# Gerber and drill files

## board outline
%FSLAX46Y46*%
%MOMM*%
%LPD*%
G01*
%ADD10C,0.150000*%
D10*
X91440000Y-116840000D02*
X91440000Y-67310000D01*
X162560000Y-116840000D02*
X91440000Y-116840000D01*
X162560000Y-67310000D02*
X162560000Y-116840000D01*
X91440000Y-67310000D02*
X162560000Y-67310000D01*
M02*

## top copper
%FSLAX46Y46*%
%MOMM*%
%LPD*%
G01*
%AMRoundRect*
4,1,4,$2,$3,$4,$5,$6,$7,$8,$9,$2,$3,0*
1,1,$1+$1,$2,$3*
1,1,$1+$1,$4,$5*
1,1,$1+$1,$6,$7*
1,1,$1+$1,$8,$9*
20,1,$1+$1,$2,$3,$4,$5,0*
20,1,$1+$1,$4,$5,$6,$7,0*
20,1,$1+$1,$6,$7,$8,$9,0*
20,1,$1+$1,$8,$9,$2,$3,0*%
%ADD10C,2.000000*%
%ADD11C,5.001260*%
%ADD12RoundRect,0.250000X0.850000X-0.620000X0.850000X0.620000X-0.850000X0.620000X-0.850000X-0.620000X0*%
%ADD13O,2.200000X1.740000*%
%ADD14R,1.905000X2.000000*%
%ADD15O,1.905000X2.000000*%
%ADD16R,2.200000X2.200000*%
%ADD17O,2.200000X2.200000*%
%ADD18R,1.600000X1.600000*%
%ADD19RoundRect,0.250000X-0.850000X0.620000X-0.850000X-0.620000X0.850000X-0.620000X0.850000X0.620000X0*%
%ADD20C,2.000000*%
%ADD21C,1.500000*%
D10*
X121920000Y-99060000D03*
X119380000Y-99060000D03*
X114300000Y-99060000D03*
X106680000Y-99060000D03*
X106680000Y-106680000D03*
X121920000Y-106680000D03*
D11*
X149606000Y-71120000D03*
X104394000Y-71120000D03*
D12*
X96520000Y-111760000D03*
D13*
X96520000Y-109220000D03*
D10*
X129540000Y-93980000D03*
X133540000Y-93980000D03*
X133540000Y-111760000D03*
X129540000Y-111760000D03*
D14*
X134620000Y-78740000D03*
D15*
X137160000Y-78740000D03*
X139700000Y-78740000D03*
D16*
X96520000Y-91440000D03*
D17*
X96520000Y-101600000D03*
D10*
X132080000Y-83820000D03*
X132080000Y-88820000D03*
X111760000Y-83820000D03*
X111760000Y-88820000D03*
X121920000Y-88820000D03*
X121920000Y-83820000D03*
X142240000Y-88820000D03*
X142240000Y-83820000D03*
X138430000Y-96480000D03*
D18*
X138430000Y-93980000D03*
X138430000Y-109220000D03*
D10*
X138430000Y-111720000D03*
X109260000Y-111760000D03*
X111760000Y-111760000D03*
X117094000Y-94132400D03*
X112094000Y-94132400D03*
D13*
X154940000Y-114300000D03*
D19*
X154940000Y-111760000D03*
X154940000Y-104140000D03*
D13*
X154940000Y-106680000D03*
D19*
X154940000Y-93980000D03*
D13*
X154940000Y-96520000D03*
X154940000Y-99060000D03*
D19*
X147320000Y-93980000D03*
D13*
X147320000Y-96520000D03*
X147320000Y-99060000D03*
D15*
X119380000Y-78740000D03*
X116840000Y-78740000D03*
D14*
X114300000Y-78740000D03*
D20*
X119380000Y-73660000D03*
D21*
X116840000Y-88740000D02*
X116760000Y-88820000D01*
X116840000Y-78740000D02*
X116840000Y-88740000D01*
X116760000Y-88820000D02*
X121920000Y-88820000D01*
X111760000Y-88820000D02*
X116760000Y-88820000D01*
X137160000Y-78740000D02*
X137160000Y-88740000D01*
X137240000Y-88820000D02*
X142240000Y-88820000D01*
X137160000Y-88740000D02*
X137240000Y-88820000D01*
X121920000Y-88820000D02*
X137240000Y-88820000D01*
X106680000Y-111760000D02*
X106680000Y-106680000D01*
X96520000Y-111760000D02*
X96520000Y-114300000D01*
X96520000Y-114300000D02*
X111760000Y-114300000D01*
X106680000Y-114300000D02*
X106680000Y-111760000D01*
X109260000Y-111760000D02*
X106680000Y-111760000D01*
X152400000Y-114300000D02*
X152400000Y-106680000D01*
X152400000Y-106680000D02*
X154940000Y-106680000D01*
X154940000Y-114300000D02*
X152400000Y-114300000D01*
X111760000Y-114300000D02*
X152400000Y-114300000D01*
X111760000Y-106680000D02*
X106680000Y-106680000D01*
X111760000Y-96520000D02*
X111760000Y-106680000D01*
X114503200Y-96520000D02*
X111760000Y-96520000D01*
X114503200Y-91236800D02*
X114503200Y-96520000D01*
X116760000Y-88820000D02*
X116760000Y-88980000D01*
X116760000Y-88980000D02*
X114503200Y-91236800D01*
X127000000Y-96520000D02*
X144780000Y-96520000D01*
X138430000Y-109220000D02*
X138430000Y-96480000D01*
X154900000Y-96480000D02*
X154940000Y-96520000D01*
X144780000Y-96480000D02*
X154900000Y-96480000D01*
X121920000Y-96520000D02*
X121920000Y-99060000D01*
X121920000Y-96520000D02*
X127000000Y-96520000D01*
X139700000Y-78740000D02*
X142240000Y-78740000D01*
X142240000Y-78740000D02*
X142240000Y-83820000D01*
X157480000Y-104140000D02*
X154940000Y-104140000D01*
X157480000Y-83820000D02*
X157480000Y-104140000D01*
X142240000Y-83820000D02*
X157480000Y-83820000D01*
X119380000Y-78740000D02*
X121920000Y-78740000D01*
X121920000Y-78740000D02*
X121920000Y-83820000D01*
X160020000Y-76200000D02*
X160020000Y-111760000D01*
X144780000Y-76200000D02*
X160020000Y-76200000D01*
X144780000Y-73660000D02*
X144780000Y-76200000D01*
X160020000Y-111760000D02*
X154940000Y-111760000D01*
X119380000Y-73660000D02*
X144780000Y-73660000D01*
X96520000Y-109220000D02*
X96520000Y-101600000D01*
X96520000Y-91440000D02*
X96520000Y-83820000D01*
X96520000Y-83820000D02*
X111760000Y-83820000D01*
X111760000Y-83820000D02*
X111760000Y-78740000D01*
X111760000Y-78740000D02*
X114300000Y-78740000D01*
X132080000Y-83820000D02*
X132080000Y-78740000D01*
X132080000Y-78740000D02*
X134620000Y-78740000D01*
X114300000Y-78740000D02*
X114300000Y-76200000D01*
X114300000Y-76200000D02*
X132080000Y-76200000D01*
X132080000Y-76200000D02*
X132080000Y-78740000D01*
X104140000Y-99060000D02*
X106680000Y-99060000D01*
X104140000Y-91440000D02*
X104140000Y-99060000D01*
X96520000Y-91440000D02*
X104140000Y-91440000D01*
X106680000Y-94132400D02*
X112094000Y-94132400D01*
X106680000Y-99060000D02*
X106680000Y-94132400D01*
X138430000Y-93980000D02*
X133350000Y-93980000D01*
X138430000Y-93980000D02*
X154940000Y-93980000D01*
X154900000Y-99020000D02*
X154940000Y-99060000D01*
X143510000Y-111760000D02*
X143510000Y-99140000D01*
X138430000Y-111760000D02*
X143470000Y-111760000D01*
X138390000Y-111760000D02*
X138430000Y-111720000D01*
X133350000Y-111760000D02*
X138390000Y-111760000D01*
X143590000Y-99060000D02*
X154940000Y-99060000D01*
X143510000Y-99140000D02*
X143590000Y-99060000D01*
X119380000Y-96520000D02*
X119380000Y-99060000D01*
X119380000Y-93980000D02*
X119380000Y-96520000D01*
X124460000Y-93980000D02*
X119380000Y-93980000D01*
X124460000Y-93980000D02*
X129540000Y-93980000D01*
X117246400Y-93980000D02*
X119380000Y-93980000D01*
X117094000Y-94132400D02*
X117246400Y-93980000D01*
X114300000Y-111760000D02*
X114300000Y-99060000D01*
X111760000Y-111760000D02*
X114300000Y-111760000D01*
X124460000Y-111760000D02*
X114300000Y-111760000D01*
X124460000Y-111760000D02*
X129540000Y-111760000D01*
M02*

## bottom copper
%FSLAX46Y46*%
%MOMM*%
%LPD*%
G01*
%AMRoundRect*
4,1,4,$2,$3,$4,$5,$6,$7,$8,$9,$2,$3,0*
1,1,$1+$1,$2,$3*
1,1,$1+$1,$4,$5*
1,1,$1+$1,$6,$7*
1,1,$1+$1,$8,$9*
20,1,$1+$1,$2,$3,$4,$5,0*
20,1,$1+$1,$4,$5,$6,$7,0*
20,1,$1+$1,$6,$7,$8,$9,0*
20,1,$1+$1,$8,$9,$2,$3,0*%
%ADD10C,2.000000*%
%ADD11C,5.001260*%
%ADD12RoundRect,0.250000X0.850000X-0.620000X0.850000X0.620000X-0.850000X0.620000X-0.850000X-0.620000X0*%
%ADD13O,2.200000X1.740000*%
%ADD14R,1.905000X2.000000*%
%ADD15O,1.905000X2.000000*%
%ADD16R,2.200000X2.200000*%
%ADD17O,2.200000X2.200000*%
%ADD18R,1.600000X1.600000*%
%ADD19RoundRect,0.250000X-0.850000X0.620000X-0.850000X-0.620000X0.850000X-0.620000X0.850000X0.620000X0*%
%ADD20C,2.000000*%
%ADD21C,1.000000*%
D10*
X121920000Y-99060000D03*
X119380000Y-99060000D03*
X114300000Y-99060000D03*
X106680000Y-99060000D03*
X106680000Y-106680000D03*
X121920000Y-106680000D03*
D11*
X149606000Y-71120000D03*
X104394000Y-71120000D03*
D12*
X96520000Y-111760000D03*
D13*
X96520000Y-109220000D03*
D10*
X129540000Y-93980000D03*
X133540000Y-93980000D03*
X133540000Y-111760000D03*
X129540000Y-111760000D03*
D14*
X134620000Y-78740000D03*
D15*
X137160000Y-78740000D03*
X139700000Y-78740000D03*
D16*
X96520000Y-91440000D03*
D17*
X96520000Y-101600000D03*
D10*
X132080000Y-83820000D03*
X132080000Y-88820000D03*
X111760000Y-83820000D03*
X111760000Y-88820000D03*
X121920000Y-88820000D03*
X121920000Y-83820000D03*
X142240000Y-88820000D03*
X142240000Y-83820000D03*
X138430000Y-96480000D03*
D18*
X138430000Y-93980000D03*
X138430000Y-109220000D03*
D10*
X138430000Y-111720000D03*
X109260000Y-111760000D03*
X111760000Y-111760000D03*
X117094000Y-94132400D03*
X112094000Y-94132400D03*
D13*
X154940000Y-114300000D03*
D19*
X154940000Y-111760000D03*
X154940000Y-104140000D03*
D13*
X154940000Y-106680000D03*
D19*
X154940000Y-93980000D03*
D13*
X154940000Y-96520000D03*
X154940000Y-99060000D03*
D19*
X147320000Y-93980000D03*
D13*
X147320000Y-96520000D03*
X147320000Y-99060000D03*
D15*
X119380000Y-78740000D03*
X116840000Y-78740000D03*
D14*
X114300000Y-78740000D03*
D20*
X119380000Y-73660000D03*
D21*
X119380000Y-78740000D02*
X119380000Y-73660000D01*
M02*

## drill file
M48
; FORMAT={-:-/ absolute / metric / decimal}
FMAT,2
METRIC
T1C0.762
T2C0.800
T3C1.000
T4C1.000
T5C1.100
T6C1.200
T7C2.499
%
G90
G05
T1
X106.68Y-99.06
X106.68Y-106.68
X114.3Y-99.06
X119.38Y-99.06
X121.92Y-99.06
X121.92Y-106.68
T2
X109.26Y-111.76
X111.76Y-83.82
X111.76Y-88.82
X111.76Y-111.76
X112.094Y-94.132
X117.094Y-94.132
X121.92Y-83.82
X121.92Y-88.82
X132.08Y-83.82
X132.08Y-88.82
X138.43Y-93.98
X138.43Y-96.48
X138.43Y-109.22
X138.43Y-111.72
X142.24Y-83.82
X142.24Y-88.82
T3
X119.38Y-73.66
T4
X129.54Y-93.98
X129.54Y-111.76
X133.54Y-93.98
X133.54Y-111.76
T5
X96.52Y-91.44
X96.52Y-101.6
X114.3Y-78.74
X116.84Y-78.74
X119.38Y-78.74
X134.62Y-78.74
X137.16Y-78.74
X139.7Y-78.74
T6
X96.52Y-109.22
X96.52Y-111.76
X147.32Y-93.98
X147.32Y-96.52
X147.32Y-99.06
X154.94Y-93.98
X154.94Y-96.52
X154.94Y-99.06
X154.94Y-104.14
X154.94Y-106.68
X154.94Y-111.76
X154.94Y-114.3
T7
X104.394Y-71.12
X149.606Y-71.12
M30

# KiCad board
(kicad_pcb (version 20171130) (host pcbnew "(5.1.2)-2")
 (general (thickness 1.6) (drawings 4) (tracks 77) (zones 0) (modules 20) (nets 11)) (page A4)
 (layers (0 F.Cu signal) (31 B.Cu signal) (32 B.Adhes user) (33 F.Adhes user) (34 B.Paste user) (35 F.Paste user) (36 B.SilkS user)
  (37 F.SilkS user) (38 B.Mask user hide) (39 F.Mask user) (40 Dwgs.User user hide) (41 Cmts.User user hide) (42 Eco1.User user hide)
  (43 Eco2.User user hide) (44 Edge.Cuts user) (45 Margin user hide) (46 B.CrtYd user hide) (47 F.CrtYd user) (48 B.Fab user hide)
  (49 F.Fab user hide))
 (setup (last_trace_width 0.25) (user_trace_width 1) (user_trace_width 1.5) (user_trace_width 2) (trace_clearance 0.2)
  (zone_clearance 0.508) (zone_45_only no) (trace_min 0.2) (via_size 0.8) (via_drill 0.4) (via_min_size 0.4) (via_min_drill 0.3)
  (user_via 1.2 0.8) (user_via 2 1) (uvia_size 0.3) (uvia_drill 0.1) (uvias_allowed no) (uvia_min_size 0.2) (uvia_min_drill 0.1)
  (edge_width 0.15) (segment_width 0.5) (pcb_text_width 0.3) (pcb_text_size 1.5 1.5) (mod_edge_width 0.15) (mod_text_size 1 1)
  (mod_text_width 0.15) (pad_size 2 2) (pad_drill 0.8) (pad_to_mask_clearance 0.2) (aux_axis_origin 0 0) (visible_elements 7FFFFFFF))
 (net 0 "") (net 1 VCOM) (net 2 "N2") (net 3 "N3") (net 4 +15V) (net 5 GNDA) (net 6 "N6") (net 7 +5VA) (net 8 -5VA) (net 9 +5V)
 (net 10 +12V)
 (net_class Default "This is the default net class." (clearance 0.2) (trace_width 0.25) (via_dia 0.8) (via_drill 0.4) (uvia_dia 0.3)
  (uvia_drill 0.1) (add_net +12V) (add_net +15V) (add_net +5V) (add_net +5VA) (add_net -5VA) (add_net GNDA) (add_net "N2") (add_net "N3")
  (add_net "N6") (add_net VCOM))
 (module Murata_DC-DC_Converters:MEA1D (layer F.Cu) (at 114.3 104.14)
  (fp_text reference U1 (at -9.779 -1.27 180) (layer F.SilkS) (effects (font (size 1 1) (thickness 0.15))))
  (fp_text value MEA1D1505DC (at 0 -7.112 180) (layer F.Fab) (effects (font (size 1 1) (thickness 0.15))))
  (pad 8 thru_hole circle (at 7.62 -5.08) (size 2 2) (drill 0.762) (layers *.Cu *.Mask) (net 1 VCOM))
  (pad 9 thru_hole circle (at 5.08 -5.08) (size 2 2) (drill 0.762) (layers *.Cu *.Mask) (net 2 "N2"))
  (pad 11 thru_hole circle (at 0 -5.08) (size 2 2) (drill 0.762) (layers *.Cu *.Mask) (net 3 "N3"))
  (pad 14 thru_hole circle (at -7.62 -5.08) (size 2 2) (drill 0.762) (layers *.Cu *.Mask) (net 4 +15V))
  (pad 1 thru_hole circle (at -7.62 2.54) (size 2 2) (drill 0.762) (layers *.Cu *.Mask) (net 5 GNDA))
  (pad 7 thru_hole circle (at 7.62 2.54) (size 2 2) (drill 0.762) (layers *.Cu *.Mask)))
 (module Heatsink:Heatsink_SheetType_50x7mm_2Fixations (layer F.Cu) (at 127 71.12) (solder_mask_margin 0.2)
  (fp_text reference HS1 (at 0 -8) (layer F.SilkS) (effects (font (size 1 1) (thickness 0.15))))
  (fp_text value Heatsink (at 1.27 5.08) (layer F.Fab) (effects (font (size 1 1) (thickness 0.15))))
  (pad 1 thru_hole circle (at 22.606 0) (size 5.00126 5.00126) (drill 2.49936) (layers *.Cu *.Mask))
  (pad 1 thru_hole circle (at -22.606 0) (size 5.00126 5.00126) (drill 2.49936) (layers *.Cu *.Mask)))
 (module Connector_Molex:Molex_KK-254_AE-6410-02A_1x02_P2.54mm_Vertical (layer F.Cu) (at 96.52 111.76 90)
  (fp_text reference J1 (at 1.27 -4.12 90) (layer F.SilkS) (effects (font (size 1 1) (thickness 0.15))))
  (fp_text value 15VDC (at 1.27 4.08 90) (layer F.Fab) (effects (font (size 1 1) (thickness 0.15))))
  (pad 1 thru_hole roundrect (at 0 0 90) (size 1.74 2.2) (drill 1.2) (layers *.Cu *.Mask) (roundrect_rratio 0.143678) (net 5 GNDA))
  (pad 2 thru_hole oval (at 2.54 0 90) (size 1.74 2.2) (drill 1.2) (layers *.Cu *.Mask) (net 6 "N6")))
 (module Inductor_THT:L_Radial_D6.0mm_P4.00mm (layer F.Cu) (at 129.54 93.98)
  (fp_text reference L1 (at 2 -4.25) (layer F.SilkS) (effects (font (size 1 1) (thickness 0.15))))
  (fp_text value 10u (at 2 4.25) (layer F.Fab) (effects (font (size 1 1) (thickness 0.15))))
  (pad 1 thru_hole circle (at 0 0) (size 2 2) (drill 1) (layers *.Cu *.Mask) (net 2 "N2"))
  (pad 2 thru_hole circle (at 4 0) (size 2 2) (drill 1) (layers *.Cu *.Mask) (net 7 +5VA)))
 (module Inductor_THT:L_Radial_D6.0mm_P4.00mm (layer F.Cu) (at 129.54 111.76)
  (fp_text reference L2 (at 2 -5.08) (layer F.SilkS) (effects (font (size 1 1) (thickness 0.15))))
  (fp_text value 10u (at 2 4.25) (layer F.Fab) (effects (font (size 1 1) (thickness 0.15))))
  (pad 2 thru_hole circle (at 4 0) (size 2 2) (drill 1) (layers *.Cu *.Mask) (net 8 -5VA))
  (pad 1 thru_hole circle (at 0 0) (size 2 2) (drill 1) (layers *.Cu *.Mask) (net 3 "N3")))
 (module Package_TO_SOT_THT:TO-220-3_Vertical (layer F.Cu) (at 134.62 78.74)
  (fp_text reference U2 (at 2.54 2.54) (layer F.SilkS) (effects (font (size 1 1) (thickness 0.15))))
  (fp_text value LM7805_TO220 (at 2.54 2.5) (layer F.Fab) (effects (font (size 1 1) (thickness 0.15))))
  (pad 1 thru_hole rect (at 0 0) (size 1.905 2) (drill 1.1) (layers *.Cu *.Mask) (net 4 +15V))
  (pad 2 thru_hole oval (at 2.54 0) (size 1.905 2) (drill 1.1) (layers *.Cu *.Mask) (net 5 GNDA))
  (pad 3 thru_hole oval (at 5.08 0) (size 1.905 2) (drill 1.1) (layers *.Cu *.Mask) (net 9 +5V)))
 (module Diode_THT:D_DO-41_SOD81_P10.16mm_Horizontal (layer F.Cu) (at 96.52 91.44 270)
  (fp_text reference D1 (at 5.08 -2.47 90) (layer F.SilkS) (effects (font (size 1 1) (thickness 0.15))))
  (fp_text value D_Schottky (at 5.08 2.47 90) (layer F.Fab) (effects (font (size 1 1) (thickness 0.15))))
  (pad 1 thru_hole rect (at 0 0 270) (size 2.2 2.2) (drill 1.1) (layers *.Cu *.Mask) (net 4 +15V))
  (pad 2 thru_hole oval (at 10.16 0 270) (size 2.2 2.2) (drill 1.1) (layers *.Cu *.Mask) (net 6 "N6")))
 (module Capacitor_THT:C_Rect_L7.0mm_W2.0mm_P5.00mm (layer F.Cu) (at 132.08 83.82 270)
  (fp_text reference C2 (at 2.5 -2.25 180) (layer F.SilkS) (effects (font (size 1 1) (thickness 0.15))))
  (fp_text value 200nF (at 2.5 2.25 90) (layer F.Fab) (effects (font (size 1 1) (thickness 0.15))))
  (pad 1 thru_hole circle (at 0 0 270) (size 2 2) (drill 0.8) (layers *.Cu *.Mask) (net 4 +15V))
  (pad 2 thru_hole circle (at 5 0 270) (size 2 2) (drill 0.8) (layers *.Cu *.Mask) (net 5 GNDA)))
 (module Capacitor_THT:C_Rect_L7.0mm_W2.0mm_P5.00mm (layer F.Cu) (at 111.76 83.82 270)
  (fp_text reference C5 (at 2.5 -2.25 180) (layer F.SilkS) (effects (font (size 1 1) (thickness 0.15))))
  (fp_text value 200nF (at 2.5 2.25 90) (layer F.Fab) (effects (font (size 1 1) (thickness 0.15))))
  (pad 1 thru_hole circle (at 0 0 270) (size 2 2) (drill 0.8) (layers *.Cu *.Mask) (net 4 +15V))
  (pad 2 thru_hole circle (at 5 0 270) (size 2 2) (drill 0.8) (layers *.Cu *.Mask) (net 5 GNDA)))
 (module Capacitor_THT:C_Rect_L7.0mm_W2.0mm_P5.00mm (layer F.Cu) (at 121.92 83.82 270)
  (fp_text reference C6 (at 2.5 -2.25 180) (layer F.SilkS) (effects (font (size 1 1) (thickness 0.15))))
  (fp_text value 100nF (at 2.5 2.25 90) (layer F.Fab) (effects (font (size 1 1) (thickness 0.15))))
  (pad 2 thru_hole circle (at 5 0 270) (size 2 2) (drill 0.8) (layers *.Cu *.Mask) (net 5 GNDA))
  (pad 1 thru_hole circle (at 0 0 270) (size 2 2) (drill 0.8) (layers *.Cu *.Mask) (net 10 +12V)))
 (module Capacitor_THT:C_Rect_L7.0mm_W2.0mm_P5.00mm (layer F.Cu) (at 142.24 83.82 270)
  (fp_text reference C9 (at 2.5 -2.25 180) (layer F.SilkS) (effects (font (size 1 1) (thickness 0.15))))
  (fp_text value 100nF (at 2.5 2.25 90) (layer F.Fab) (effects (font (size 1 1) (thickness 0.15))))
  (pad 2 thru_hole circle (at 5 0 270) (size 2 2) (drill 0.8) (layers *.Cu *.Mask) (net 5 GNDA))
  (pad 1 thru_hole circle (at 0 0 270) (size 2 2) (drill 0.8) (layers *.Cu *.Mask) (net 9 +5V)))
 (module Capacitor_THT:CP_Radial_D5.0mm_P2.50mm (layer F.Cu) (at 138.43 93.98 270)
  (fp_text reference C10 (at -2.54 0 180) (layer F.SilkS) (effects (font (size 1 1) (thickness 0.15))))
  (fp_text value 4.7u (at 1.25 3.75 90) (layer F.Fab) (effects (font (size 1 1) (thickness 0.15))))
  (pad 2 thru_hole circle (at 2.5 0 270) (size 2 2) (drill 0.8) (layers *.Cu *.Mask) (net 1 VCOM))
  (pad 1 thru_hole rect (at 0 0 270) (size 1.6 1.6) (drill 0.8) (layers *.Cu *.Mask) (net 7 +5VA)))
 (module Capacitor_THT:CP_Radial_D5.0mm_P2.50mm (layer F.Cu) (at 138.43 109.22 270)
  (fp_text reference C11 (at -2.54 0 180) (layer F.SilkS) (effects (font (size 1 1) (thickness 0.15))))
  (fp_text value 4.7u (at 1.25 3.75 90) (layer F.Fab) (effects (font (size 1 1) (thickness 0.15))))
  (pad 1 thru_hole rect (at 0 0 270) (size 1.6 1.6) (drill 0.8) (layers *.Cu *.Mask) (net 1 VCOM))
  (pad 2 thru_hole circle (at 2.5 0 270) (size 2 2) (drill 0.8) (layers *.Cu *.Mask) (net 8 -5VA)))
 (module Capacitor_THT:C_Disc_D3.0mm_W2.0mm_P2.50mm (layer F.Cu) (at 111.76 111.76 180)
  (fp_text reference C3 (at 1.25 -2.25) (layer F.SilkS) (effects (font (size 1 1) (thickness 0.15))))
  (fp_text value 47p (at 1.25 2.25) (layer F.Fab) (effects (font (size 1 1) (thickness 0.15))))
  (pad 2 thru_hole circle (at 2.5 0 180) (size 2 2) (drill 0.8) (layers *.Cu *.Mask) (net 5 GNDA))
  (pad 1 thru_hole circle (at 0 0 180) (size 2 2) (drill 0.8) (layers *.Cu *.Mask) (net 3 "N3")))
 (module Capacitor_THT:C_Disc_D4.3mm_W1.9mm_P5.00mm (layer F.Cu) (at 117.094 94.1324 180)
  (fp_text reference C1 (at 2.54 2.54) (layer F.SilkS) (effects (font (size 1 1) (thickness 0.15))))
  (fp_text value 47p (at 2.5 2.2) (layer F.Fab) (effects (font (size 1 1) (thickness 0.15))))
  (pad 1 thru_hole circle (at 0 0 180) (size 2 2) (drill 0.8) (layers *.Cu *.Mask) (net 2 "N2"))
  (pad 2 thru_hole circle (at 5 0 180) (size 2 2) (drill 0.8) (layers *.Cu *.Mask) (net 4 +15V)))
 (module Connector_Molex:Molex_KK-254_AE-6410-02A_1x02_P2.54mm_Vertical (layer F.Cu) (at 154.94 111.76 270)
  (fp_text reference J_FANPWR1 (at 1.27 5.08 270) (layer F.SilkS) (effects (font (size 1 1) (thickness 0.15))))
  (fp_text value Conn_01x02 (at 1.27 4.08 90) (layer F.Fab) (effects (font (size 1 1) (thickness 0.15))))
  (pad 2 thru_hole oval (at 2.54 0 270) (size 1.74 2.2) (drill 1.2) (layers *.Cu *.Mask) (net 5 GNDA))
  (pad 1 thru_hole roundrect (at 0 0 270) (size 1.74 2.2) (drill 1.2) (layers *.Cu *.Mask) (roundrect_rratio 0.143678) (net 10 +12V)))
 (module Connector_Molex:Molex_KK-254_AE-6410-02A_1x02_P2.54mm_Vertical (layer F.Cu) (at 154.94 104.14 270)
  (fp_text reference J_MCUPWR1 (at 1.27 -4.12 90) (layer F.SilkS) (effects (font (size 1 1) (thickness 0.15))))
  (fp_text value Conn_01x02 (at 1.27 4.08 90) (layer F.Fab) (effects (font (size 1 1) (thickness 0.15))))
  (pad 1 thru_hole roundrect (at 0 0 270) (size 1.74 2.2) (drill 1.2) (layers *.Cu *.Mask) (roundrect_rratio 0.143678) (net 9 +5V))
  (pad 2 thru_hole oval (at 2.54 0 270) (size 1.74 2.2) (drill 1.2) (layers *.Cu *.Mask) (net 5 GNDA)))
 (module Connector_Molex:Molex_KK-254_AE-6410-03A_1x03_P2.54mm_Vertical (layer F.Cu) (at 154.94 93.98 270)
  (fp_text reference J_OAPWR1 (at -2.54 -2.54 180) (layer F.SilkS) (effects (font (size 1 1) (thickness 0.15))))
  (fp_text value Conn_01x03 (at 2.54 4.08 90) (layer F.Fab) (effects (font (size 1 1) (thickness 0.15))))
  (pad 1 thru_hole roundrect (at 0 0 270) (size 1.74 2.2) (drill 1.2) (layers *.Cu *.Mask) (roundrect_rratio 0.143678) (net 7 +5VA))
  (pad 2 thru_hole oval (at 2.54 0 270) (size 1.74 2.2) (drill 1.2) (layers *.Cu *.Mask) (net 1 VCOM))
  (pad 3 thru_hole oval (at 5.08 0 270) (size 1.74 2.2) (drill 1.2) (layers *.Cu *.Mask) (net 8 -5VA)))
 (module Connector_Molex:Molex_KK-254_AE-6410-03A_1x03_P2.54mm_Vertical (layer F.Cu) (at 147.32 93.98 270)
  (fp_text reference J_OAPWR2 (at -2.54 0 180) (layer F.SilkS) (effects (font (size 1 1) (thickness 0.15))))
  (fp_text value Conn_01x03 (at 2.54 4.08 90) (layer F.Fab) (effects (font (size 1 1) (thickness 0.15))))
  (pad 1 thru_hole roundrect (at 0 0 270) (size 1.74 2.2) (drill 1.2) (layers *.Cu *.Mask) (roundrect_rratio 0.143678) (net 7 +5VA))
  (pad 2 thru_hole oval (at 2.54 0 270) (size 1.74 2.2) (drill 1.2) (layers *.Cu *.Mask) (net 1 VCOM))
  (pad 3 thru_hole oval (at 5.08 0 270) (size 1.74 2.2) (drill 1.2) (layers *.Cu *.Mask) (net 8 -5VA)))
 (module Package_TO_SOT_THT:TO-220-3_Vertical (layer F.Cu) (at 114.3 78.74)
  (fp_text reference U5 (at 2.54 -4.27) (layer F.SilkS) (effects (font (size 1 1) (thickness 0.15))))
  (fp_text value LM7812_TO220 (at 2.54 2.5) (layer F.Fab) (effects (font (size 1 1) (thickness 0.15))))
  (pad 3 thru_hole oval (at 5.08 0) (size 1.905 2) (drill 1.1) (layers *.Cu *.Mask) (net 10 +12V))
  (pad 2 thru_hole oval (at 2.54 0) (size 1.905 2) (drill 1.1) (layers *.Cu *.Mask) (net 5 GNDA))
  (pad 1 thru_hole rect (at 0 0) (size 1.905 2) (drill 1.1) (layers *.Cu *.Mask) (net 4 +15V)))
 (gr_line (start 91.44 116.84) (end 91.44 67.31) (layer Edge.Cuts) (width 0.15))
 (gr_line (start 162.56 116.84) (end 91.44 116.84) (layer Edge.Cuts) (width 0.15))
 (gr_line (start 162.56 67.31) (end 162.56 116.84) (layer Edge.Cuts) (width 0.15))
 (gr_line (start 91.44 67.31) (end 162.56 67.31) (layer Edge.Cuts) (width 0.15))
 (segment (start 116.84 88.74) (end 116.76 88.82) (width 1.5) (layer F.Cu) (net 5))
 (segment (start 116.84 78.74) (end 116.84 88.74) (width 1.5) (layer F.Cu) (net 5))
 (segment (start 116.76 88.82) (end 121.92 88.82) (width 1.5) (layer F.Cu) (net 5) (status 20))
 (segment (start 111.76 88.82) (end 116.76 88.82) (width 1.5) (layer F.Cu) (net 5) (status 10))
 (segment (start 137.16 78.74) (end 137.16 88.74) (width 1.5) (layer F.Cu) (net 5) (status 10))
 (segment (start 137.24 88.82) (end 142.24 88.82) (width 1.5) (layer F.Cu) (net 5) (status 20))
 (segment (start 137.16 88.74) (end 137.24 88.82) (width 1.5) (layer F.Cu) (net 5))
 (segment (start 121.92 88.82) (end 137.24 88.82) (width 1.5) (layer F.Cu) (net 5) (status 10))
 (segment (start 106.68 111.76) (end 106.68 106.68) (width 1.5) (layer F.Cu) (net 5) (status 20))
 (segment (start 96.52 111.76) (end 96.52 114.3) (width 1.5) (layer F.Cu) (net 5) (status 10))
 (segment (start 96.52 114.3) (end 111.76 114.3) (width 1.5) (layer F.Cu) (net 5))
 (segment (start 106.68 114.3) (end 106.68 111.76) (width 1.5) (layer F.Cu) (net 5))
 (segment (start 109.26 111.76) (end 106.68 111.76) (width 1.5) (layer F.Cu) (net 5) (status 10))
 (segment (start 152.4 114.3) (end 152.4 106.68) (width 1.5) (layer F.Cu) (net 5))
 (segment (start 152.4 106.68) (end 154.94 106.68) (width 1.5) (layer F.Cu) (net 5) (status 20))
 (segment (start 154.94 114.3) (end 152.4 114.3) (width 1.5) (layer F.Cu) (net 5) (status 10))
 (segment (start 111.76 114.3) (end 152.4 114.3) (width 1.5) (layer F.Cu) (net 5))
 (segment (start 111.76 106.68) (end 106.68 106.68) (width 1.5) (layer F.Cu) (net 5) (status 20))
 (segment (start 111.76 96.52) (end 111.76 106.68) (width 1.5) (layer F.Cu) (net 5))
 (segment (start 114.5032 96.52) (end 111.76 96.52) (width 1.5) (layer F.Cu) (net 5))
 (segment (start 114.5032 91.2368) (end 114.5032 96.52) (width 1.5) (layer F.Cu) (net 5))
 (segment (start 116.76 88.82) (end 116.76 88.98) (width 1.5) (layer F.Cu) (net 5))
 (segment (start 116.76 88.98) (end 114.5032 91.2368) (width 1.5) (layer F.Cu) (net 5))
 (segment (start 127 96.52) (end 144.78 96.52) (width 1.5) (layer F.Cu) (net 1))
 (segment (start 138.43 109.22) (end 138.43 96.48) (width 1.5) (layer F.Cu) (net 1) (status 30))
 (segment (start 154.9 96.48) (end 154.94 96.52) (width 1.5) (layer F.Cu) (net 1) (status 30))
 (segment (start 144.78 96.48) (end 154.9 96.48) (width 1.5) (layer F.Cu) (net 1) (status 20))
 (segment (start 121.92 96.52) (end 121.92 99.06) (width 1.5) (layer F.Cu) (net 1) (status 20))
 (segment (start 121.92 96.52) (end 127 96.52) (width 1.5) (layer F.Cu) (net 1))
 (segment (start 139.7 78.74) (end 142.24 78.74) (width 1.5) (layer F.Cu) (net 9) (status 10))
 (segment (start 142.24 78.74) (end 142.24 83.82) (width 1.5) (layer F.Cu) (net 9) (status 20))
 (segment (start 157.48 104.14) (end 154.94 104.14) (width 1.5) (layer F.Cu) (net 9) (status 20))
 (segment (start 157.48 83.82) (end 157.48 104.14) (width 1.5) (layer F.Cu) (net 9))
 (segment (start 142.24 83.82) (end 157.48 83.82) (width 1.5) (layer F.Cu) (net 9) (status 10))
 (segment (start 119.38 78.74) (end 121.92 78.74) (width 1.5) (layer F.Cu) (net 10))
 (segment (start 121.92 78.74) (end 121.92 83.82) (width 1.5) (layer F.Cu) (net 10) (status 20))
 (segment (start 119.38 78.74) (end 119.38 73.66) (width 1) (layer B.Cu) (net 10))
 (via (at 119.38 73.66) (size 2) (drill 1) (layers F.Cu B.Cu) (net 10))
 (segment (start 160.02 76.2) (end 160.02 111.76) (width 1.5) (layer F.Cu) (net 10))
 (segment (start 144.78 76.2) (end 160.02 76.2) (width 1.5) (layer F.Cu) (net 10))
 (segment (start 144.78 73.66) (end 144.78 76.2) (width 1.5) (layer F.Cu) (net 10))
 (segment (start 160.02 111.76) (end 154.94 111.76) (width 1.5) (layer F.Cu) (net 10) (status 20))
 (segment (start 119.38 73.66) (end 144.78 73.66) (width 1.5) (layer F.Cu) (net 10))
 (segment (start 96.52 109.22) (end 96.52 101.6) (width 1.5) (layer F.Cu) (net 6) (status 30))
 (segment (start 96.52 91.44) (end 96.52 83.82) (width 1.5) (layer F.Cu) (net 4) (status 10))
 (segment (start 96.52 83.82) (end 111.76 83.82) (width 1.5) (layer F.Cu) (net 4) (status 20))
 (segment (start 111.76 83.82) (end 111.76 78.74) (width 1.5) (layer F.Cu) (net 4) (status 10))
 (segment (start 111.76 78.74) (end 114.3 78.74) (width 1.5) (layer F.Cu) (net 4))
 (segment (start 132.08 83.82) (end 132.08 78.74) (width 1.5) (layer F.Cu) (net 4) (status 10))
 (segment (start 132.08 78.74) (end 134.62 78.74) (width 1.5) (layer F.Cu) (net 4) (status 20))
 (segment (start 114.3 78.74) (end 114.3 76.2) (width 1.5) (layer F.Cu) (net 4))
 (segment (start 114.3 76.2) (end 132.08 76.2) (width 1.5) (layer F.Cu) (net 4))
 (segment (start 132.08 76.2) (end 132.08 78.74) (width 1.5) (layer F.Cu) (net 4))
 (segment (start 104.14 99.06) (end 106.68 99.06) (width 1.5) (layer F.Cu) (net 4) (status 20))
 (segment (start 104.14 91.44) (end 104.14 99.06) (width 1.5) (layer F.Cu) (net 4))
 (segment (start 96.52 91.44) (end 104.14 91.44) (width 1.5) (layer F.Cu) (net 4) (status 10))
 (segment (start 106.68 94.1324) (end 112.094 94.1324) (width 1.5) (layer F.Cu) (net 4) (status 20))
 (segment (start 106.68 99.06) (end 106.68 94.1324) (width 1.5) (layer F.Cu) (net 4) (status 10))
 (segment (start 138.43 93.98) (end 133.35 93.98) (width 1.5) (layer F.Cu) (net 7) (status 30))
 (segment (start 138.43 93.98) (end 154.94 93.98) (width 1.5) (layer F.Cu) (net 7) (status 30))
 (segment (start 154.9 99.02) (end 154.94 99.06) (width 1.5) (layer F.Cu) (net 8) (status 30))
 (segment (start 143.51 111.76) (end 143.51 99.14) (width 1.5) (layer F.Cu) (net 8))
 (segment (start 138.43 111.76) (end 143.47 111.76) (width 1.5) (layer F.Cu) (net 8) (status 10))
 (segment (start 138.39 111.76) (end 138.43 111.72) (width 1.5) (layer F.Cu) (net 8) (status 30))
 (segment (start 133.35 111.76) (end 138.39 111.76) (width 1.5) (layer F.Cu) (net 8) (status 30))
 (segment (start 143.59 99.06) (end 154.94 99.06) (width 1.5) (layer F.Cu) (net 8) (status 20))
 (segment (start 143.51 99.14) (end 143.59 99.06) (width 1.5) (layer F.Cu) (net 8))
 (segment (start 119.38 96.52) (end 119.38 99.06) (width 1.5) (layer F.Cu) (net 2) (status 20))
 (segment (start 119.38 93.98) (end 119.38 96.52) (width 1.5) (layer F.Cu) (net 2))
 (segment (start 124.46 93.98) (end 119.38 93.98) (width 1.5) (layer F.Cu) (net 2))
 (segment (start 124.46 93.98) (end 129.54 93.98) (width 1.5) (layer F.Cu) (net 2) (status 20))
 (segment (start 117.2464 93.98) (end 119.38 93.98) (width 1.5) (layer F.Cu) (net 2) (status 10))
 (segment (start 117.094 94.1324) (end 117.2464 93.98) (width 1.5) (layer F.Cu) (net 2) (status 30))
 (segment (start 114.3 111.76) (end 114.3 99.06) (width 1.5) (layer F.Cu) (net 3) (status 20))
 (segment (start 111.76 111.76) (end 114.3 111.76) (width 1.5) (layer F.Cu) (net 3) (status 10))
 (segment (start 124.46 111.76) (end 114.3 111.76) (width 1.5) (layer F.Cu) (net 3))
 (segment (start 124.46 111.76) (end 129.54 111.76) (width 1.5) (layer F.Cu) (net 3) (status 20)))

